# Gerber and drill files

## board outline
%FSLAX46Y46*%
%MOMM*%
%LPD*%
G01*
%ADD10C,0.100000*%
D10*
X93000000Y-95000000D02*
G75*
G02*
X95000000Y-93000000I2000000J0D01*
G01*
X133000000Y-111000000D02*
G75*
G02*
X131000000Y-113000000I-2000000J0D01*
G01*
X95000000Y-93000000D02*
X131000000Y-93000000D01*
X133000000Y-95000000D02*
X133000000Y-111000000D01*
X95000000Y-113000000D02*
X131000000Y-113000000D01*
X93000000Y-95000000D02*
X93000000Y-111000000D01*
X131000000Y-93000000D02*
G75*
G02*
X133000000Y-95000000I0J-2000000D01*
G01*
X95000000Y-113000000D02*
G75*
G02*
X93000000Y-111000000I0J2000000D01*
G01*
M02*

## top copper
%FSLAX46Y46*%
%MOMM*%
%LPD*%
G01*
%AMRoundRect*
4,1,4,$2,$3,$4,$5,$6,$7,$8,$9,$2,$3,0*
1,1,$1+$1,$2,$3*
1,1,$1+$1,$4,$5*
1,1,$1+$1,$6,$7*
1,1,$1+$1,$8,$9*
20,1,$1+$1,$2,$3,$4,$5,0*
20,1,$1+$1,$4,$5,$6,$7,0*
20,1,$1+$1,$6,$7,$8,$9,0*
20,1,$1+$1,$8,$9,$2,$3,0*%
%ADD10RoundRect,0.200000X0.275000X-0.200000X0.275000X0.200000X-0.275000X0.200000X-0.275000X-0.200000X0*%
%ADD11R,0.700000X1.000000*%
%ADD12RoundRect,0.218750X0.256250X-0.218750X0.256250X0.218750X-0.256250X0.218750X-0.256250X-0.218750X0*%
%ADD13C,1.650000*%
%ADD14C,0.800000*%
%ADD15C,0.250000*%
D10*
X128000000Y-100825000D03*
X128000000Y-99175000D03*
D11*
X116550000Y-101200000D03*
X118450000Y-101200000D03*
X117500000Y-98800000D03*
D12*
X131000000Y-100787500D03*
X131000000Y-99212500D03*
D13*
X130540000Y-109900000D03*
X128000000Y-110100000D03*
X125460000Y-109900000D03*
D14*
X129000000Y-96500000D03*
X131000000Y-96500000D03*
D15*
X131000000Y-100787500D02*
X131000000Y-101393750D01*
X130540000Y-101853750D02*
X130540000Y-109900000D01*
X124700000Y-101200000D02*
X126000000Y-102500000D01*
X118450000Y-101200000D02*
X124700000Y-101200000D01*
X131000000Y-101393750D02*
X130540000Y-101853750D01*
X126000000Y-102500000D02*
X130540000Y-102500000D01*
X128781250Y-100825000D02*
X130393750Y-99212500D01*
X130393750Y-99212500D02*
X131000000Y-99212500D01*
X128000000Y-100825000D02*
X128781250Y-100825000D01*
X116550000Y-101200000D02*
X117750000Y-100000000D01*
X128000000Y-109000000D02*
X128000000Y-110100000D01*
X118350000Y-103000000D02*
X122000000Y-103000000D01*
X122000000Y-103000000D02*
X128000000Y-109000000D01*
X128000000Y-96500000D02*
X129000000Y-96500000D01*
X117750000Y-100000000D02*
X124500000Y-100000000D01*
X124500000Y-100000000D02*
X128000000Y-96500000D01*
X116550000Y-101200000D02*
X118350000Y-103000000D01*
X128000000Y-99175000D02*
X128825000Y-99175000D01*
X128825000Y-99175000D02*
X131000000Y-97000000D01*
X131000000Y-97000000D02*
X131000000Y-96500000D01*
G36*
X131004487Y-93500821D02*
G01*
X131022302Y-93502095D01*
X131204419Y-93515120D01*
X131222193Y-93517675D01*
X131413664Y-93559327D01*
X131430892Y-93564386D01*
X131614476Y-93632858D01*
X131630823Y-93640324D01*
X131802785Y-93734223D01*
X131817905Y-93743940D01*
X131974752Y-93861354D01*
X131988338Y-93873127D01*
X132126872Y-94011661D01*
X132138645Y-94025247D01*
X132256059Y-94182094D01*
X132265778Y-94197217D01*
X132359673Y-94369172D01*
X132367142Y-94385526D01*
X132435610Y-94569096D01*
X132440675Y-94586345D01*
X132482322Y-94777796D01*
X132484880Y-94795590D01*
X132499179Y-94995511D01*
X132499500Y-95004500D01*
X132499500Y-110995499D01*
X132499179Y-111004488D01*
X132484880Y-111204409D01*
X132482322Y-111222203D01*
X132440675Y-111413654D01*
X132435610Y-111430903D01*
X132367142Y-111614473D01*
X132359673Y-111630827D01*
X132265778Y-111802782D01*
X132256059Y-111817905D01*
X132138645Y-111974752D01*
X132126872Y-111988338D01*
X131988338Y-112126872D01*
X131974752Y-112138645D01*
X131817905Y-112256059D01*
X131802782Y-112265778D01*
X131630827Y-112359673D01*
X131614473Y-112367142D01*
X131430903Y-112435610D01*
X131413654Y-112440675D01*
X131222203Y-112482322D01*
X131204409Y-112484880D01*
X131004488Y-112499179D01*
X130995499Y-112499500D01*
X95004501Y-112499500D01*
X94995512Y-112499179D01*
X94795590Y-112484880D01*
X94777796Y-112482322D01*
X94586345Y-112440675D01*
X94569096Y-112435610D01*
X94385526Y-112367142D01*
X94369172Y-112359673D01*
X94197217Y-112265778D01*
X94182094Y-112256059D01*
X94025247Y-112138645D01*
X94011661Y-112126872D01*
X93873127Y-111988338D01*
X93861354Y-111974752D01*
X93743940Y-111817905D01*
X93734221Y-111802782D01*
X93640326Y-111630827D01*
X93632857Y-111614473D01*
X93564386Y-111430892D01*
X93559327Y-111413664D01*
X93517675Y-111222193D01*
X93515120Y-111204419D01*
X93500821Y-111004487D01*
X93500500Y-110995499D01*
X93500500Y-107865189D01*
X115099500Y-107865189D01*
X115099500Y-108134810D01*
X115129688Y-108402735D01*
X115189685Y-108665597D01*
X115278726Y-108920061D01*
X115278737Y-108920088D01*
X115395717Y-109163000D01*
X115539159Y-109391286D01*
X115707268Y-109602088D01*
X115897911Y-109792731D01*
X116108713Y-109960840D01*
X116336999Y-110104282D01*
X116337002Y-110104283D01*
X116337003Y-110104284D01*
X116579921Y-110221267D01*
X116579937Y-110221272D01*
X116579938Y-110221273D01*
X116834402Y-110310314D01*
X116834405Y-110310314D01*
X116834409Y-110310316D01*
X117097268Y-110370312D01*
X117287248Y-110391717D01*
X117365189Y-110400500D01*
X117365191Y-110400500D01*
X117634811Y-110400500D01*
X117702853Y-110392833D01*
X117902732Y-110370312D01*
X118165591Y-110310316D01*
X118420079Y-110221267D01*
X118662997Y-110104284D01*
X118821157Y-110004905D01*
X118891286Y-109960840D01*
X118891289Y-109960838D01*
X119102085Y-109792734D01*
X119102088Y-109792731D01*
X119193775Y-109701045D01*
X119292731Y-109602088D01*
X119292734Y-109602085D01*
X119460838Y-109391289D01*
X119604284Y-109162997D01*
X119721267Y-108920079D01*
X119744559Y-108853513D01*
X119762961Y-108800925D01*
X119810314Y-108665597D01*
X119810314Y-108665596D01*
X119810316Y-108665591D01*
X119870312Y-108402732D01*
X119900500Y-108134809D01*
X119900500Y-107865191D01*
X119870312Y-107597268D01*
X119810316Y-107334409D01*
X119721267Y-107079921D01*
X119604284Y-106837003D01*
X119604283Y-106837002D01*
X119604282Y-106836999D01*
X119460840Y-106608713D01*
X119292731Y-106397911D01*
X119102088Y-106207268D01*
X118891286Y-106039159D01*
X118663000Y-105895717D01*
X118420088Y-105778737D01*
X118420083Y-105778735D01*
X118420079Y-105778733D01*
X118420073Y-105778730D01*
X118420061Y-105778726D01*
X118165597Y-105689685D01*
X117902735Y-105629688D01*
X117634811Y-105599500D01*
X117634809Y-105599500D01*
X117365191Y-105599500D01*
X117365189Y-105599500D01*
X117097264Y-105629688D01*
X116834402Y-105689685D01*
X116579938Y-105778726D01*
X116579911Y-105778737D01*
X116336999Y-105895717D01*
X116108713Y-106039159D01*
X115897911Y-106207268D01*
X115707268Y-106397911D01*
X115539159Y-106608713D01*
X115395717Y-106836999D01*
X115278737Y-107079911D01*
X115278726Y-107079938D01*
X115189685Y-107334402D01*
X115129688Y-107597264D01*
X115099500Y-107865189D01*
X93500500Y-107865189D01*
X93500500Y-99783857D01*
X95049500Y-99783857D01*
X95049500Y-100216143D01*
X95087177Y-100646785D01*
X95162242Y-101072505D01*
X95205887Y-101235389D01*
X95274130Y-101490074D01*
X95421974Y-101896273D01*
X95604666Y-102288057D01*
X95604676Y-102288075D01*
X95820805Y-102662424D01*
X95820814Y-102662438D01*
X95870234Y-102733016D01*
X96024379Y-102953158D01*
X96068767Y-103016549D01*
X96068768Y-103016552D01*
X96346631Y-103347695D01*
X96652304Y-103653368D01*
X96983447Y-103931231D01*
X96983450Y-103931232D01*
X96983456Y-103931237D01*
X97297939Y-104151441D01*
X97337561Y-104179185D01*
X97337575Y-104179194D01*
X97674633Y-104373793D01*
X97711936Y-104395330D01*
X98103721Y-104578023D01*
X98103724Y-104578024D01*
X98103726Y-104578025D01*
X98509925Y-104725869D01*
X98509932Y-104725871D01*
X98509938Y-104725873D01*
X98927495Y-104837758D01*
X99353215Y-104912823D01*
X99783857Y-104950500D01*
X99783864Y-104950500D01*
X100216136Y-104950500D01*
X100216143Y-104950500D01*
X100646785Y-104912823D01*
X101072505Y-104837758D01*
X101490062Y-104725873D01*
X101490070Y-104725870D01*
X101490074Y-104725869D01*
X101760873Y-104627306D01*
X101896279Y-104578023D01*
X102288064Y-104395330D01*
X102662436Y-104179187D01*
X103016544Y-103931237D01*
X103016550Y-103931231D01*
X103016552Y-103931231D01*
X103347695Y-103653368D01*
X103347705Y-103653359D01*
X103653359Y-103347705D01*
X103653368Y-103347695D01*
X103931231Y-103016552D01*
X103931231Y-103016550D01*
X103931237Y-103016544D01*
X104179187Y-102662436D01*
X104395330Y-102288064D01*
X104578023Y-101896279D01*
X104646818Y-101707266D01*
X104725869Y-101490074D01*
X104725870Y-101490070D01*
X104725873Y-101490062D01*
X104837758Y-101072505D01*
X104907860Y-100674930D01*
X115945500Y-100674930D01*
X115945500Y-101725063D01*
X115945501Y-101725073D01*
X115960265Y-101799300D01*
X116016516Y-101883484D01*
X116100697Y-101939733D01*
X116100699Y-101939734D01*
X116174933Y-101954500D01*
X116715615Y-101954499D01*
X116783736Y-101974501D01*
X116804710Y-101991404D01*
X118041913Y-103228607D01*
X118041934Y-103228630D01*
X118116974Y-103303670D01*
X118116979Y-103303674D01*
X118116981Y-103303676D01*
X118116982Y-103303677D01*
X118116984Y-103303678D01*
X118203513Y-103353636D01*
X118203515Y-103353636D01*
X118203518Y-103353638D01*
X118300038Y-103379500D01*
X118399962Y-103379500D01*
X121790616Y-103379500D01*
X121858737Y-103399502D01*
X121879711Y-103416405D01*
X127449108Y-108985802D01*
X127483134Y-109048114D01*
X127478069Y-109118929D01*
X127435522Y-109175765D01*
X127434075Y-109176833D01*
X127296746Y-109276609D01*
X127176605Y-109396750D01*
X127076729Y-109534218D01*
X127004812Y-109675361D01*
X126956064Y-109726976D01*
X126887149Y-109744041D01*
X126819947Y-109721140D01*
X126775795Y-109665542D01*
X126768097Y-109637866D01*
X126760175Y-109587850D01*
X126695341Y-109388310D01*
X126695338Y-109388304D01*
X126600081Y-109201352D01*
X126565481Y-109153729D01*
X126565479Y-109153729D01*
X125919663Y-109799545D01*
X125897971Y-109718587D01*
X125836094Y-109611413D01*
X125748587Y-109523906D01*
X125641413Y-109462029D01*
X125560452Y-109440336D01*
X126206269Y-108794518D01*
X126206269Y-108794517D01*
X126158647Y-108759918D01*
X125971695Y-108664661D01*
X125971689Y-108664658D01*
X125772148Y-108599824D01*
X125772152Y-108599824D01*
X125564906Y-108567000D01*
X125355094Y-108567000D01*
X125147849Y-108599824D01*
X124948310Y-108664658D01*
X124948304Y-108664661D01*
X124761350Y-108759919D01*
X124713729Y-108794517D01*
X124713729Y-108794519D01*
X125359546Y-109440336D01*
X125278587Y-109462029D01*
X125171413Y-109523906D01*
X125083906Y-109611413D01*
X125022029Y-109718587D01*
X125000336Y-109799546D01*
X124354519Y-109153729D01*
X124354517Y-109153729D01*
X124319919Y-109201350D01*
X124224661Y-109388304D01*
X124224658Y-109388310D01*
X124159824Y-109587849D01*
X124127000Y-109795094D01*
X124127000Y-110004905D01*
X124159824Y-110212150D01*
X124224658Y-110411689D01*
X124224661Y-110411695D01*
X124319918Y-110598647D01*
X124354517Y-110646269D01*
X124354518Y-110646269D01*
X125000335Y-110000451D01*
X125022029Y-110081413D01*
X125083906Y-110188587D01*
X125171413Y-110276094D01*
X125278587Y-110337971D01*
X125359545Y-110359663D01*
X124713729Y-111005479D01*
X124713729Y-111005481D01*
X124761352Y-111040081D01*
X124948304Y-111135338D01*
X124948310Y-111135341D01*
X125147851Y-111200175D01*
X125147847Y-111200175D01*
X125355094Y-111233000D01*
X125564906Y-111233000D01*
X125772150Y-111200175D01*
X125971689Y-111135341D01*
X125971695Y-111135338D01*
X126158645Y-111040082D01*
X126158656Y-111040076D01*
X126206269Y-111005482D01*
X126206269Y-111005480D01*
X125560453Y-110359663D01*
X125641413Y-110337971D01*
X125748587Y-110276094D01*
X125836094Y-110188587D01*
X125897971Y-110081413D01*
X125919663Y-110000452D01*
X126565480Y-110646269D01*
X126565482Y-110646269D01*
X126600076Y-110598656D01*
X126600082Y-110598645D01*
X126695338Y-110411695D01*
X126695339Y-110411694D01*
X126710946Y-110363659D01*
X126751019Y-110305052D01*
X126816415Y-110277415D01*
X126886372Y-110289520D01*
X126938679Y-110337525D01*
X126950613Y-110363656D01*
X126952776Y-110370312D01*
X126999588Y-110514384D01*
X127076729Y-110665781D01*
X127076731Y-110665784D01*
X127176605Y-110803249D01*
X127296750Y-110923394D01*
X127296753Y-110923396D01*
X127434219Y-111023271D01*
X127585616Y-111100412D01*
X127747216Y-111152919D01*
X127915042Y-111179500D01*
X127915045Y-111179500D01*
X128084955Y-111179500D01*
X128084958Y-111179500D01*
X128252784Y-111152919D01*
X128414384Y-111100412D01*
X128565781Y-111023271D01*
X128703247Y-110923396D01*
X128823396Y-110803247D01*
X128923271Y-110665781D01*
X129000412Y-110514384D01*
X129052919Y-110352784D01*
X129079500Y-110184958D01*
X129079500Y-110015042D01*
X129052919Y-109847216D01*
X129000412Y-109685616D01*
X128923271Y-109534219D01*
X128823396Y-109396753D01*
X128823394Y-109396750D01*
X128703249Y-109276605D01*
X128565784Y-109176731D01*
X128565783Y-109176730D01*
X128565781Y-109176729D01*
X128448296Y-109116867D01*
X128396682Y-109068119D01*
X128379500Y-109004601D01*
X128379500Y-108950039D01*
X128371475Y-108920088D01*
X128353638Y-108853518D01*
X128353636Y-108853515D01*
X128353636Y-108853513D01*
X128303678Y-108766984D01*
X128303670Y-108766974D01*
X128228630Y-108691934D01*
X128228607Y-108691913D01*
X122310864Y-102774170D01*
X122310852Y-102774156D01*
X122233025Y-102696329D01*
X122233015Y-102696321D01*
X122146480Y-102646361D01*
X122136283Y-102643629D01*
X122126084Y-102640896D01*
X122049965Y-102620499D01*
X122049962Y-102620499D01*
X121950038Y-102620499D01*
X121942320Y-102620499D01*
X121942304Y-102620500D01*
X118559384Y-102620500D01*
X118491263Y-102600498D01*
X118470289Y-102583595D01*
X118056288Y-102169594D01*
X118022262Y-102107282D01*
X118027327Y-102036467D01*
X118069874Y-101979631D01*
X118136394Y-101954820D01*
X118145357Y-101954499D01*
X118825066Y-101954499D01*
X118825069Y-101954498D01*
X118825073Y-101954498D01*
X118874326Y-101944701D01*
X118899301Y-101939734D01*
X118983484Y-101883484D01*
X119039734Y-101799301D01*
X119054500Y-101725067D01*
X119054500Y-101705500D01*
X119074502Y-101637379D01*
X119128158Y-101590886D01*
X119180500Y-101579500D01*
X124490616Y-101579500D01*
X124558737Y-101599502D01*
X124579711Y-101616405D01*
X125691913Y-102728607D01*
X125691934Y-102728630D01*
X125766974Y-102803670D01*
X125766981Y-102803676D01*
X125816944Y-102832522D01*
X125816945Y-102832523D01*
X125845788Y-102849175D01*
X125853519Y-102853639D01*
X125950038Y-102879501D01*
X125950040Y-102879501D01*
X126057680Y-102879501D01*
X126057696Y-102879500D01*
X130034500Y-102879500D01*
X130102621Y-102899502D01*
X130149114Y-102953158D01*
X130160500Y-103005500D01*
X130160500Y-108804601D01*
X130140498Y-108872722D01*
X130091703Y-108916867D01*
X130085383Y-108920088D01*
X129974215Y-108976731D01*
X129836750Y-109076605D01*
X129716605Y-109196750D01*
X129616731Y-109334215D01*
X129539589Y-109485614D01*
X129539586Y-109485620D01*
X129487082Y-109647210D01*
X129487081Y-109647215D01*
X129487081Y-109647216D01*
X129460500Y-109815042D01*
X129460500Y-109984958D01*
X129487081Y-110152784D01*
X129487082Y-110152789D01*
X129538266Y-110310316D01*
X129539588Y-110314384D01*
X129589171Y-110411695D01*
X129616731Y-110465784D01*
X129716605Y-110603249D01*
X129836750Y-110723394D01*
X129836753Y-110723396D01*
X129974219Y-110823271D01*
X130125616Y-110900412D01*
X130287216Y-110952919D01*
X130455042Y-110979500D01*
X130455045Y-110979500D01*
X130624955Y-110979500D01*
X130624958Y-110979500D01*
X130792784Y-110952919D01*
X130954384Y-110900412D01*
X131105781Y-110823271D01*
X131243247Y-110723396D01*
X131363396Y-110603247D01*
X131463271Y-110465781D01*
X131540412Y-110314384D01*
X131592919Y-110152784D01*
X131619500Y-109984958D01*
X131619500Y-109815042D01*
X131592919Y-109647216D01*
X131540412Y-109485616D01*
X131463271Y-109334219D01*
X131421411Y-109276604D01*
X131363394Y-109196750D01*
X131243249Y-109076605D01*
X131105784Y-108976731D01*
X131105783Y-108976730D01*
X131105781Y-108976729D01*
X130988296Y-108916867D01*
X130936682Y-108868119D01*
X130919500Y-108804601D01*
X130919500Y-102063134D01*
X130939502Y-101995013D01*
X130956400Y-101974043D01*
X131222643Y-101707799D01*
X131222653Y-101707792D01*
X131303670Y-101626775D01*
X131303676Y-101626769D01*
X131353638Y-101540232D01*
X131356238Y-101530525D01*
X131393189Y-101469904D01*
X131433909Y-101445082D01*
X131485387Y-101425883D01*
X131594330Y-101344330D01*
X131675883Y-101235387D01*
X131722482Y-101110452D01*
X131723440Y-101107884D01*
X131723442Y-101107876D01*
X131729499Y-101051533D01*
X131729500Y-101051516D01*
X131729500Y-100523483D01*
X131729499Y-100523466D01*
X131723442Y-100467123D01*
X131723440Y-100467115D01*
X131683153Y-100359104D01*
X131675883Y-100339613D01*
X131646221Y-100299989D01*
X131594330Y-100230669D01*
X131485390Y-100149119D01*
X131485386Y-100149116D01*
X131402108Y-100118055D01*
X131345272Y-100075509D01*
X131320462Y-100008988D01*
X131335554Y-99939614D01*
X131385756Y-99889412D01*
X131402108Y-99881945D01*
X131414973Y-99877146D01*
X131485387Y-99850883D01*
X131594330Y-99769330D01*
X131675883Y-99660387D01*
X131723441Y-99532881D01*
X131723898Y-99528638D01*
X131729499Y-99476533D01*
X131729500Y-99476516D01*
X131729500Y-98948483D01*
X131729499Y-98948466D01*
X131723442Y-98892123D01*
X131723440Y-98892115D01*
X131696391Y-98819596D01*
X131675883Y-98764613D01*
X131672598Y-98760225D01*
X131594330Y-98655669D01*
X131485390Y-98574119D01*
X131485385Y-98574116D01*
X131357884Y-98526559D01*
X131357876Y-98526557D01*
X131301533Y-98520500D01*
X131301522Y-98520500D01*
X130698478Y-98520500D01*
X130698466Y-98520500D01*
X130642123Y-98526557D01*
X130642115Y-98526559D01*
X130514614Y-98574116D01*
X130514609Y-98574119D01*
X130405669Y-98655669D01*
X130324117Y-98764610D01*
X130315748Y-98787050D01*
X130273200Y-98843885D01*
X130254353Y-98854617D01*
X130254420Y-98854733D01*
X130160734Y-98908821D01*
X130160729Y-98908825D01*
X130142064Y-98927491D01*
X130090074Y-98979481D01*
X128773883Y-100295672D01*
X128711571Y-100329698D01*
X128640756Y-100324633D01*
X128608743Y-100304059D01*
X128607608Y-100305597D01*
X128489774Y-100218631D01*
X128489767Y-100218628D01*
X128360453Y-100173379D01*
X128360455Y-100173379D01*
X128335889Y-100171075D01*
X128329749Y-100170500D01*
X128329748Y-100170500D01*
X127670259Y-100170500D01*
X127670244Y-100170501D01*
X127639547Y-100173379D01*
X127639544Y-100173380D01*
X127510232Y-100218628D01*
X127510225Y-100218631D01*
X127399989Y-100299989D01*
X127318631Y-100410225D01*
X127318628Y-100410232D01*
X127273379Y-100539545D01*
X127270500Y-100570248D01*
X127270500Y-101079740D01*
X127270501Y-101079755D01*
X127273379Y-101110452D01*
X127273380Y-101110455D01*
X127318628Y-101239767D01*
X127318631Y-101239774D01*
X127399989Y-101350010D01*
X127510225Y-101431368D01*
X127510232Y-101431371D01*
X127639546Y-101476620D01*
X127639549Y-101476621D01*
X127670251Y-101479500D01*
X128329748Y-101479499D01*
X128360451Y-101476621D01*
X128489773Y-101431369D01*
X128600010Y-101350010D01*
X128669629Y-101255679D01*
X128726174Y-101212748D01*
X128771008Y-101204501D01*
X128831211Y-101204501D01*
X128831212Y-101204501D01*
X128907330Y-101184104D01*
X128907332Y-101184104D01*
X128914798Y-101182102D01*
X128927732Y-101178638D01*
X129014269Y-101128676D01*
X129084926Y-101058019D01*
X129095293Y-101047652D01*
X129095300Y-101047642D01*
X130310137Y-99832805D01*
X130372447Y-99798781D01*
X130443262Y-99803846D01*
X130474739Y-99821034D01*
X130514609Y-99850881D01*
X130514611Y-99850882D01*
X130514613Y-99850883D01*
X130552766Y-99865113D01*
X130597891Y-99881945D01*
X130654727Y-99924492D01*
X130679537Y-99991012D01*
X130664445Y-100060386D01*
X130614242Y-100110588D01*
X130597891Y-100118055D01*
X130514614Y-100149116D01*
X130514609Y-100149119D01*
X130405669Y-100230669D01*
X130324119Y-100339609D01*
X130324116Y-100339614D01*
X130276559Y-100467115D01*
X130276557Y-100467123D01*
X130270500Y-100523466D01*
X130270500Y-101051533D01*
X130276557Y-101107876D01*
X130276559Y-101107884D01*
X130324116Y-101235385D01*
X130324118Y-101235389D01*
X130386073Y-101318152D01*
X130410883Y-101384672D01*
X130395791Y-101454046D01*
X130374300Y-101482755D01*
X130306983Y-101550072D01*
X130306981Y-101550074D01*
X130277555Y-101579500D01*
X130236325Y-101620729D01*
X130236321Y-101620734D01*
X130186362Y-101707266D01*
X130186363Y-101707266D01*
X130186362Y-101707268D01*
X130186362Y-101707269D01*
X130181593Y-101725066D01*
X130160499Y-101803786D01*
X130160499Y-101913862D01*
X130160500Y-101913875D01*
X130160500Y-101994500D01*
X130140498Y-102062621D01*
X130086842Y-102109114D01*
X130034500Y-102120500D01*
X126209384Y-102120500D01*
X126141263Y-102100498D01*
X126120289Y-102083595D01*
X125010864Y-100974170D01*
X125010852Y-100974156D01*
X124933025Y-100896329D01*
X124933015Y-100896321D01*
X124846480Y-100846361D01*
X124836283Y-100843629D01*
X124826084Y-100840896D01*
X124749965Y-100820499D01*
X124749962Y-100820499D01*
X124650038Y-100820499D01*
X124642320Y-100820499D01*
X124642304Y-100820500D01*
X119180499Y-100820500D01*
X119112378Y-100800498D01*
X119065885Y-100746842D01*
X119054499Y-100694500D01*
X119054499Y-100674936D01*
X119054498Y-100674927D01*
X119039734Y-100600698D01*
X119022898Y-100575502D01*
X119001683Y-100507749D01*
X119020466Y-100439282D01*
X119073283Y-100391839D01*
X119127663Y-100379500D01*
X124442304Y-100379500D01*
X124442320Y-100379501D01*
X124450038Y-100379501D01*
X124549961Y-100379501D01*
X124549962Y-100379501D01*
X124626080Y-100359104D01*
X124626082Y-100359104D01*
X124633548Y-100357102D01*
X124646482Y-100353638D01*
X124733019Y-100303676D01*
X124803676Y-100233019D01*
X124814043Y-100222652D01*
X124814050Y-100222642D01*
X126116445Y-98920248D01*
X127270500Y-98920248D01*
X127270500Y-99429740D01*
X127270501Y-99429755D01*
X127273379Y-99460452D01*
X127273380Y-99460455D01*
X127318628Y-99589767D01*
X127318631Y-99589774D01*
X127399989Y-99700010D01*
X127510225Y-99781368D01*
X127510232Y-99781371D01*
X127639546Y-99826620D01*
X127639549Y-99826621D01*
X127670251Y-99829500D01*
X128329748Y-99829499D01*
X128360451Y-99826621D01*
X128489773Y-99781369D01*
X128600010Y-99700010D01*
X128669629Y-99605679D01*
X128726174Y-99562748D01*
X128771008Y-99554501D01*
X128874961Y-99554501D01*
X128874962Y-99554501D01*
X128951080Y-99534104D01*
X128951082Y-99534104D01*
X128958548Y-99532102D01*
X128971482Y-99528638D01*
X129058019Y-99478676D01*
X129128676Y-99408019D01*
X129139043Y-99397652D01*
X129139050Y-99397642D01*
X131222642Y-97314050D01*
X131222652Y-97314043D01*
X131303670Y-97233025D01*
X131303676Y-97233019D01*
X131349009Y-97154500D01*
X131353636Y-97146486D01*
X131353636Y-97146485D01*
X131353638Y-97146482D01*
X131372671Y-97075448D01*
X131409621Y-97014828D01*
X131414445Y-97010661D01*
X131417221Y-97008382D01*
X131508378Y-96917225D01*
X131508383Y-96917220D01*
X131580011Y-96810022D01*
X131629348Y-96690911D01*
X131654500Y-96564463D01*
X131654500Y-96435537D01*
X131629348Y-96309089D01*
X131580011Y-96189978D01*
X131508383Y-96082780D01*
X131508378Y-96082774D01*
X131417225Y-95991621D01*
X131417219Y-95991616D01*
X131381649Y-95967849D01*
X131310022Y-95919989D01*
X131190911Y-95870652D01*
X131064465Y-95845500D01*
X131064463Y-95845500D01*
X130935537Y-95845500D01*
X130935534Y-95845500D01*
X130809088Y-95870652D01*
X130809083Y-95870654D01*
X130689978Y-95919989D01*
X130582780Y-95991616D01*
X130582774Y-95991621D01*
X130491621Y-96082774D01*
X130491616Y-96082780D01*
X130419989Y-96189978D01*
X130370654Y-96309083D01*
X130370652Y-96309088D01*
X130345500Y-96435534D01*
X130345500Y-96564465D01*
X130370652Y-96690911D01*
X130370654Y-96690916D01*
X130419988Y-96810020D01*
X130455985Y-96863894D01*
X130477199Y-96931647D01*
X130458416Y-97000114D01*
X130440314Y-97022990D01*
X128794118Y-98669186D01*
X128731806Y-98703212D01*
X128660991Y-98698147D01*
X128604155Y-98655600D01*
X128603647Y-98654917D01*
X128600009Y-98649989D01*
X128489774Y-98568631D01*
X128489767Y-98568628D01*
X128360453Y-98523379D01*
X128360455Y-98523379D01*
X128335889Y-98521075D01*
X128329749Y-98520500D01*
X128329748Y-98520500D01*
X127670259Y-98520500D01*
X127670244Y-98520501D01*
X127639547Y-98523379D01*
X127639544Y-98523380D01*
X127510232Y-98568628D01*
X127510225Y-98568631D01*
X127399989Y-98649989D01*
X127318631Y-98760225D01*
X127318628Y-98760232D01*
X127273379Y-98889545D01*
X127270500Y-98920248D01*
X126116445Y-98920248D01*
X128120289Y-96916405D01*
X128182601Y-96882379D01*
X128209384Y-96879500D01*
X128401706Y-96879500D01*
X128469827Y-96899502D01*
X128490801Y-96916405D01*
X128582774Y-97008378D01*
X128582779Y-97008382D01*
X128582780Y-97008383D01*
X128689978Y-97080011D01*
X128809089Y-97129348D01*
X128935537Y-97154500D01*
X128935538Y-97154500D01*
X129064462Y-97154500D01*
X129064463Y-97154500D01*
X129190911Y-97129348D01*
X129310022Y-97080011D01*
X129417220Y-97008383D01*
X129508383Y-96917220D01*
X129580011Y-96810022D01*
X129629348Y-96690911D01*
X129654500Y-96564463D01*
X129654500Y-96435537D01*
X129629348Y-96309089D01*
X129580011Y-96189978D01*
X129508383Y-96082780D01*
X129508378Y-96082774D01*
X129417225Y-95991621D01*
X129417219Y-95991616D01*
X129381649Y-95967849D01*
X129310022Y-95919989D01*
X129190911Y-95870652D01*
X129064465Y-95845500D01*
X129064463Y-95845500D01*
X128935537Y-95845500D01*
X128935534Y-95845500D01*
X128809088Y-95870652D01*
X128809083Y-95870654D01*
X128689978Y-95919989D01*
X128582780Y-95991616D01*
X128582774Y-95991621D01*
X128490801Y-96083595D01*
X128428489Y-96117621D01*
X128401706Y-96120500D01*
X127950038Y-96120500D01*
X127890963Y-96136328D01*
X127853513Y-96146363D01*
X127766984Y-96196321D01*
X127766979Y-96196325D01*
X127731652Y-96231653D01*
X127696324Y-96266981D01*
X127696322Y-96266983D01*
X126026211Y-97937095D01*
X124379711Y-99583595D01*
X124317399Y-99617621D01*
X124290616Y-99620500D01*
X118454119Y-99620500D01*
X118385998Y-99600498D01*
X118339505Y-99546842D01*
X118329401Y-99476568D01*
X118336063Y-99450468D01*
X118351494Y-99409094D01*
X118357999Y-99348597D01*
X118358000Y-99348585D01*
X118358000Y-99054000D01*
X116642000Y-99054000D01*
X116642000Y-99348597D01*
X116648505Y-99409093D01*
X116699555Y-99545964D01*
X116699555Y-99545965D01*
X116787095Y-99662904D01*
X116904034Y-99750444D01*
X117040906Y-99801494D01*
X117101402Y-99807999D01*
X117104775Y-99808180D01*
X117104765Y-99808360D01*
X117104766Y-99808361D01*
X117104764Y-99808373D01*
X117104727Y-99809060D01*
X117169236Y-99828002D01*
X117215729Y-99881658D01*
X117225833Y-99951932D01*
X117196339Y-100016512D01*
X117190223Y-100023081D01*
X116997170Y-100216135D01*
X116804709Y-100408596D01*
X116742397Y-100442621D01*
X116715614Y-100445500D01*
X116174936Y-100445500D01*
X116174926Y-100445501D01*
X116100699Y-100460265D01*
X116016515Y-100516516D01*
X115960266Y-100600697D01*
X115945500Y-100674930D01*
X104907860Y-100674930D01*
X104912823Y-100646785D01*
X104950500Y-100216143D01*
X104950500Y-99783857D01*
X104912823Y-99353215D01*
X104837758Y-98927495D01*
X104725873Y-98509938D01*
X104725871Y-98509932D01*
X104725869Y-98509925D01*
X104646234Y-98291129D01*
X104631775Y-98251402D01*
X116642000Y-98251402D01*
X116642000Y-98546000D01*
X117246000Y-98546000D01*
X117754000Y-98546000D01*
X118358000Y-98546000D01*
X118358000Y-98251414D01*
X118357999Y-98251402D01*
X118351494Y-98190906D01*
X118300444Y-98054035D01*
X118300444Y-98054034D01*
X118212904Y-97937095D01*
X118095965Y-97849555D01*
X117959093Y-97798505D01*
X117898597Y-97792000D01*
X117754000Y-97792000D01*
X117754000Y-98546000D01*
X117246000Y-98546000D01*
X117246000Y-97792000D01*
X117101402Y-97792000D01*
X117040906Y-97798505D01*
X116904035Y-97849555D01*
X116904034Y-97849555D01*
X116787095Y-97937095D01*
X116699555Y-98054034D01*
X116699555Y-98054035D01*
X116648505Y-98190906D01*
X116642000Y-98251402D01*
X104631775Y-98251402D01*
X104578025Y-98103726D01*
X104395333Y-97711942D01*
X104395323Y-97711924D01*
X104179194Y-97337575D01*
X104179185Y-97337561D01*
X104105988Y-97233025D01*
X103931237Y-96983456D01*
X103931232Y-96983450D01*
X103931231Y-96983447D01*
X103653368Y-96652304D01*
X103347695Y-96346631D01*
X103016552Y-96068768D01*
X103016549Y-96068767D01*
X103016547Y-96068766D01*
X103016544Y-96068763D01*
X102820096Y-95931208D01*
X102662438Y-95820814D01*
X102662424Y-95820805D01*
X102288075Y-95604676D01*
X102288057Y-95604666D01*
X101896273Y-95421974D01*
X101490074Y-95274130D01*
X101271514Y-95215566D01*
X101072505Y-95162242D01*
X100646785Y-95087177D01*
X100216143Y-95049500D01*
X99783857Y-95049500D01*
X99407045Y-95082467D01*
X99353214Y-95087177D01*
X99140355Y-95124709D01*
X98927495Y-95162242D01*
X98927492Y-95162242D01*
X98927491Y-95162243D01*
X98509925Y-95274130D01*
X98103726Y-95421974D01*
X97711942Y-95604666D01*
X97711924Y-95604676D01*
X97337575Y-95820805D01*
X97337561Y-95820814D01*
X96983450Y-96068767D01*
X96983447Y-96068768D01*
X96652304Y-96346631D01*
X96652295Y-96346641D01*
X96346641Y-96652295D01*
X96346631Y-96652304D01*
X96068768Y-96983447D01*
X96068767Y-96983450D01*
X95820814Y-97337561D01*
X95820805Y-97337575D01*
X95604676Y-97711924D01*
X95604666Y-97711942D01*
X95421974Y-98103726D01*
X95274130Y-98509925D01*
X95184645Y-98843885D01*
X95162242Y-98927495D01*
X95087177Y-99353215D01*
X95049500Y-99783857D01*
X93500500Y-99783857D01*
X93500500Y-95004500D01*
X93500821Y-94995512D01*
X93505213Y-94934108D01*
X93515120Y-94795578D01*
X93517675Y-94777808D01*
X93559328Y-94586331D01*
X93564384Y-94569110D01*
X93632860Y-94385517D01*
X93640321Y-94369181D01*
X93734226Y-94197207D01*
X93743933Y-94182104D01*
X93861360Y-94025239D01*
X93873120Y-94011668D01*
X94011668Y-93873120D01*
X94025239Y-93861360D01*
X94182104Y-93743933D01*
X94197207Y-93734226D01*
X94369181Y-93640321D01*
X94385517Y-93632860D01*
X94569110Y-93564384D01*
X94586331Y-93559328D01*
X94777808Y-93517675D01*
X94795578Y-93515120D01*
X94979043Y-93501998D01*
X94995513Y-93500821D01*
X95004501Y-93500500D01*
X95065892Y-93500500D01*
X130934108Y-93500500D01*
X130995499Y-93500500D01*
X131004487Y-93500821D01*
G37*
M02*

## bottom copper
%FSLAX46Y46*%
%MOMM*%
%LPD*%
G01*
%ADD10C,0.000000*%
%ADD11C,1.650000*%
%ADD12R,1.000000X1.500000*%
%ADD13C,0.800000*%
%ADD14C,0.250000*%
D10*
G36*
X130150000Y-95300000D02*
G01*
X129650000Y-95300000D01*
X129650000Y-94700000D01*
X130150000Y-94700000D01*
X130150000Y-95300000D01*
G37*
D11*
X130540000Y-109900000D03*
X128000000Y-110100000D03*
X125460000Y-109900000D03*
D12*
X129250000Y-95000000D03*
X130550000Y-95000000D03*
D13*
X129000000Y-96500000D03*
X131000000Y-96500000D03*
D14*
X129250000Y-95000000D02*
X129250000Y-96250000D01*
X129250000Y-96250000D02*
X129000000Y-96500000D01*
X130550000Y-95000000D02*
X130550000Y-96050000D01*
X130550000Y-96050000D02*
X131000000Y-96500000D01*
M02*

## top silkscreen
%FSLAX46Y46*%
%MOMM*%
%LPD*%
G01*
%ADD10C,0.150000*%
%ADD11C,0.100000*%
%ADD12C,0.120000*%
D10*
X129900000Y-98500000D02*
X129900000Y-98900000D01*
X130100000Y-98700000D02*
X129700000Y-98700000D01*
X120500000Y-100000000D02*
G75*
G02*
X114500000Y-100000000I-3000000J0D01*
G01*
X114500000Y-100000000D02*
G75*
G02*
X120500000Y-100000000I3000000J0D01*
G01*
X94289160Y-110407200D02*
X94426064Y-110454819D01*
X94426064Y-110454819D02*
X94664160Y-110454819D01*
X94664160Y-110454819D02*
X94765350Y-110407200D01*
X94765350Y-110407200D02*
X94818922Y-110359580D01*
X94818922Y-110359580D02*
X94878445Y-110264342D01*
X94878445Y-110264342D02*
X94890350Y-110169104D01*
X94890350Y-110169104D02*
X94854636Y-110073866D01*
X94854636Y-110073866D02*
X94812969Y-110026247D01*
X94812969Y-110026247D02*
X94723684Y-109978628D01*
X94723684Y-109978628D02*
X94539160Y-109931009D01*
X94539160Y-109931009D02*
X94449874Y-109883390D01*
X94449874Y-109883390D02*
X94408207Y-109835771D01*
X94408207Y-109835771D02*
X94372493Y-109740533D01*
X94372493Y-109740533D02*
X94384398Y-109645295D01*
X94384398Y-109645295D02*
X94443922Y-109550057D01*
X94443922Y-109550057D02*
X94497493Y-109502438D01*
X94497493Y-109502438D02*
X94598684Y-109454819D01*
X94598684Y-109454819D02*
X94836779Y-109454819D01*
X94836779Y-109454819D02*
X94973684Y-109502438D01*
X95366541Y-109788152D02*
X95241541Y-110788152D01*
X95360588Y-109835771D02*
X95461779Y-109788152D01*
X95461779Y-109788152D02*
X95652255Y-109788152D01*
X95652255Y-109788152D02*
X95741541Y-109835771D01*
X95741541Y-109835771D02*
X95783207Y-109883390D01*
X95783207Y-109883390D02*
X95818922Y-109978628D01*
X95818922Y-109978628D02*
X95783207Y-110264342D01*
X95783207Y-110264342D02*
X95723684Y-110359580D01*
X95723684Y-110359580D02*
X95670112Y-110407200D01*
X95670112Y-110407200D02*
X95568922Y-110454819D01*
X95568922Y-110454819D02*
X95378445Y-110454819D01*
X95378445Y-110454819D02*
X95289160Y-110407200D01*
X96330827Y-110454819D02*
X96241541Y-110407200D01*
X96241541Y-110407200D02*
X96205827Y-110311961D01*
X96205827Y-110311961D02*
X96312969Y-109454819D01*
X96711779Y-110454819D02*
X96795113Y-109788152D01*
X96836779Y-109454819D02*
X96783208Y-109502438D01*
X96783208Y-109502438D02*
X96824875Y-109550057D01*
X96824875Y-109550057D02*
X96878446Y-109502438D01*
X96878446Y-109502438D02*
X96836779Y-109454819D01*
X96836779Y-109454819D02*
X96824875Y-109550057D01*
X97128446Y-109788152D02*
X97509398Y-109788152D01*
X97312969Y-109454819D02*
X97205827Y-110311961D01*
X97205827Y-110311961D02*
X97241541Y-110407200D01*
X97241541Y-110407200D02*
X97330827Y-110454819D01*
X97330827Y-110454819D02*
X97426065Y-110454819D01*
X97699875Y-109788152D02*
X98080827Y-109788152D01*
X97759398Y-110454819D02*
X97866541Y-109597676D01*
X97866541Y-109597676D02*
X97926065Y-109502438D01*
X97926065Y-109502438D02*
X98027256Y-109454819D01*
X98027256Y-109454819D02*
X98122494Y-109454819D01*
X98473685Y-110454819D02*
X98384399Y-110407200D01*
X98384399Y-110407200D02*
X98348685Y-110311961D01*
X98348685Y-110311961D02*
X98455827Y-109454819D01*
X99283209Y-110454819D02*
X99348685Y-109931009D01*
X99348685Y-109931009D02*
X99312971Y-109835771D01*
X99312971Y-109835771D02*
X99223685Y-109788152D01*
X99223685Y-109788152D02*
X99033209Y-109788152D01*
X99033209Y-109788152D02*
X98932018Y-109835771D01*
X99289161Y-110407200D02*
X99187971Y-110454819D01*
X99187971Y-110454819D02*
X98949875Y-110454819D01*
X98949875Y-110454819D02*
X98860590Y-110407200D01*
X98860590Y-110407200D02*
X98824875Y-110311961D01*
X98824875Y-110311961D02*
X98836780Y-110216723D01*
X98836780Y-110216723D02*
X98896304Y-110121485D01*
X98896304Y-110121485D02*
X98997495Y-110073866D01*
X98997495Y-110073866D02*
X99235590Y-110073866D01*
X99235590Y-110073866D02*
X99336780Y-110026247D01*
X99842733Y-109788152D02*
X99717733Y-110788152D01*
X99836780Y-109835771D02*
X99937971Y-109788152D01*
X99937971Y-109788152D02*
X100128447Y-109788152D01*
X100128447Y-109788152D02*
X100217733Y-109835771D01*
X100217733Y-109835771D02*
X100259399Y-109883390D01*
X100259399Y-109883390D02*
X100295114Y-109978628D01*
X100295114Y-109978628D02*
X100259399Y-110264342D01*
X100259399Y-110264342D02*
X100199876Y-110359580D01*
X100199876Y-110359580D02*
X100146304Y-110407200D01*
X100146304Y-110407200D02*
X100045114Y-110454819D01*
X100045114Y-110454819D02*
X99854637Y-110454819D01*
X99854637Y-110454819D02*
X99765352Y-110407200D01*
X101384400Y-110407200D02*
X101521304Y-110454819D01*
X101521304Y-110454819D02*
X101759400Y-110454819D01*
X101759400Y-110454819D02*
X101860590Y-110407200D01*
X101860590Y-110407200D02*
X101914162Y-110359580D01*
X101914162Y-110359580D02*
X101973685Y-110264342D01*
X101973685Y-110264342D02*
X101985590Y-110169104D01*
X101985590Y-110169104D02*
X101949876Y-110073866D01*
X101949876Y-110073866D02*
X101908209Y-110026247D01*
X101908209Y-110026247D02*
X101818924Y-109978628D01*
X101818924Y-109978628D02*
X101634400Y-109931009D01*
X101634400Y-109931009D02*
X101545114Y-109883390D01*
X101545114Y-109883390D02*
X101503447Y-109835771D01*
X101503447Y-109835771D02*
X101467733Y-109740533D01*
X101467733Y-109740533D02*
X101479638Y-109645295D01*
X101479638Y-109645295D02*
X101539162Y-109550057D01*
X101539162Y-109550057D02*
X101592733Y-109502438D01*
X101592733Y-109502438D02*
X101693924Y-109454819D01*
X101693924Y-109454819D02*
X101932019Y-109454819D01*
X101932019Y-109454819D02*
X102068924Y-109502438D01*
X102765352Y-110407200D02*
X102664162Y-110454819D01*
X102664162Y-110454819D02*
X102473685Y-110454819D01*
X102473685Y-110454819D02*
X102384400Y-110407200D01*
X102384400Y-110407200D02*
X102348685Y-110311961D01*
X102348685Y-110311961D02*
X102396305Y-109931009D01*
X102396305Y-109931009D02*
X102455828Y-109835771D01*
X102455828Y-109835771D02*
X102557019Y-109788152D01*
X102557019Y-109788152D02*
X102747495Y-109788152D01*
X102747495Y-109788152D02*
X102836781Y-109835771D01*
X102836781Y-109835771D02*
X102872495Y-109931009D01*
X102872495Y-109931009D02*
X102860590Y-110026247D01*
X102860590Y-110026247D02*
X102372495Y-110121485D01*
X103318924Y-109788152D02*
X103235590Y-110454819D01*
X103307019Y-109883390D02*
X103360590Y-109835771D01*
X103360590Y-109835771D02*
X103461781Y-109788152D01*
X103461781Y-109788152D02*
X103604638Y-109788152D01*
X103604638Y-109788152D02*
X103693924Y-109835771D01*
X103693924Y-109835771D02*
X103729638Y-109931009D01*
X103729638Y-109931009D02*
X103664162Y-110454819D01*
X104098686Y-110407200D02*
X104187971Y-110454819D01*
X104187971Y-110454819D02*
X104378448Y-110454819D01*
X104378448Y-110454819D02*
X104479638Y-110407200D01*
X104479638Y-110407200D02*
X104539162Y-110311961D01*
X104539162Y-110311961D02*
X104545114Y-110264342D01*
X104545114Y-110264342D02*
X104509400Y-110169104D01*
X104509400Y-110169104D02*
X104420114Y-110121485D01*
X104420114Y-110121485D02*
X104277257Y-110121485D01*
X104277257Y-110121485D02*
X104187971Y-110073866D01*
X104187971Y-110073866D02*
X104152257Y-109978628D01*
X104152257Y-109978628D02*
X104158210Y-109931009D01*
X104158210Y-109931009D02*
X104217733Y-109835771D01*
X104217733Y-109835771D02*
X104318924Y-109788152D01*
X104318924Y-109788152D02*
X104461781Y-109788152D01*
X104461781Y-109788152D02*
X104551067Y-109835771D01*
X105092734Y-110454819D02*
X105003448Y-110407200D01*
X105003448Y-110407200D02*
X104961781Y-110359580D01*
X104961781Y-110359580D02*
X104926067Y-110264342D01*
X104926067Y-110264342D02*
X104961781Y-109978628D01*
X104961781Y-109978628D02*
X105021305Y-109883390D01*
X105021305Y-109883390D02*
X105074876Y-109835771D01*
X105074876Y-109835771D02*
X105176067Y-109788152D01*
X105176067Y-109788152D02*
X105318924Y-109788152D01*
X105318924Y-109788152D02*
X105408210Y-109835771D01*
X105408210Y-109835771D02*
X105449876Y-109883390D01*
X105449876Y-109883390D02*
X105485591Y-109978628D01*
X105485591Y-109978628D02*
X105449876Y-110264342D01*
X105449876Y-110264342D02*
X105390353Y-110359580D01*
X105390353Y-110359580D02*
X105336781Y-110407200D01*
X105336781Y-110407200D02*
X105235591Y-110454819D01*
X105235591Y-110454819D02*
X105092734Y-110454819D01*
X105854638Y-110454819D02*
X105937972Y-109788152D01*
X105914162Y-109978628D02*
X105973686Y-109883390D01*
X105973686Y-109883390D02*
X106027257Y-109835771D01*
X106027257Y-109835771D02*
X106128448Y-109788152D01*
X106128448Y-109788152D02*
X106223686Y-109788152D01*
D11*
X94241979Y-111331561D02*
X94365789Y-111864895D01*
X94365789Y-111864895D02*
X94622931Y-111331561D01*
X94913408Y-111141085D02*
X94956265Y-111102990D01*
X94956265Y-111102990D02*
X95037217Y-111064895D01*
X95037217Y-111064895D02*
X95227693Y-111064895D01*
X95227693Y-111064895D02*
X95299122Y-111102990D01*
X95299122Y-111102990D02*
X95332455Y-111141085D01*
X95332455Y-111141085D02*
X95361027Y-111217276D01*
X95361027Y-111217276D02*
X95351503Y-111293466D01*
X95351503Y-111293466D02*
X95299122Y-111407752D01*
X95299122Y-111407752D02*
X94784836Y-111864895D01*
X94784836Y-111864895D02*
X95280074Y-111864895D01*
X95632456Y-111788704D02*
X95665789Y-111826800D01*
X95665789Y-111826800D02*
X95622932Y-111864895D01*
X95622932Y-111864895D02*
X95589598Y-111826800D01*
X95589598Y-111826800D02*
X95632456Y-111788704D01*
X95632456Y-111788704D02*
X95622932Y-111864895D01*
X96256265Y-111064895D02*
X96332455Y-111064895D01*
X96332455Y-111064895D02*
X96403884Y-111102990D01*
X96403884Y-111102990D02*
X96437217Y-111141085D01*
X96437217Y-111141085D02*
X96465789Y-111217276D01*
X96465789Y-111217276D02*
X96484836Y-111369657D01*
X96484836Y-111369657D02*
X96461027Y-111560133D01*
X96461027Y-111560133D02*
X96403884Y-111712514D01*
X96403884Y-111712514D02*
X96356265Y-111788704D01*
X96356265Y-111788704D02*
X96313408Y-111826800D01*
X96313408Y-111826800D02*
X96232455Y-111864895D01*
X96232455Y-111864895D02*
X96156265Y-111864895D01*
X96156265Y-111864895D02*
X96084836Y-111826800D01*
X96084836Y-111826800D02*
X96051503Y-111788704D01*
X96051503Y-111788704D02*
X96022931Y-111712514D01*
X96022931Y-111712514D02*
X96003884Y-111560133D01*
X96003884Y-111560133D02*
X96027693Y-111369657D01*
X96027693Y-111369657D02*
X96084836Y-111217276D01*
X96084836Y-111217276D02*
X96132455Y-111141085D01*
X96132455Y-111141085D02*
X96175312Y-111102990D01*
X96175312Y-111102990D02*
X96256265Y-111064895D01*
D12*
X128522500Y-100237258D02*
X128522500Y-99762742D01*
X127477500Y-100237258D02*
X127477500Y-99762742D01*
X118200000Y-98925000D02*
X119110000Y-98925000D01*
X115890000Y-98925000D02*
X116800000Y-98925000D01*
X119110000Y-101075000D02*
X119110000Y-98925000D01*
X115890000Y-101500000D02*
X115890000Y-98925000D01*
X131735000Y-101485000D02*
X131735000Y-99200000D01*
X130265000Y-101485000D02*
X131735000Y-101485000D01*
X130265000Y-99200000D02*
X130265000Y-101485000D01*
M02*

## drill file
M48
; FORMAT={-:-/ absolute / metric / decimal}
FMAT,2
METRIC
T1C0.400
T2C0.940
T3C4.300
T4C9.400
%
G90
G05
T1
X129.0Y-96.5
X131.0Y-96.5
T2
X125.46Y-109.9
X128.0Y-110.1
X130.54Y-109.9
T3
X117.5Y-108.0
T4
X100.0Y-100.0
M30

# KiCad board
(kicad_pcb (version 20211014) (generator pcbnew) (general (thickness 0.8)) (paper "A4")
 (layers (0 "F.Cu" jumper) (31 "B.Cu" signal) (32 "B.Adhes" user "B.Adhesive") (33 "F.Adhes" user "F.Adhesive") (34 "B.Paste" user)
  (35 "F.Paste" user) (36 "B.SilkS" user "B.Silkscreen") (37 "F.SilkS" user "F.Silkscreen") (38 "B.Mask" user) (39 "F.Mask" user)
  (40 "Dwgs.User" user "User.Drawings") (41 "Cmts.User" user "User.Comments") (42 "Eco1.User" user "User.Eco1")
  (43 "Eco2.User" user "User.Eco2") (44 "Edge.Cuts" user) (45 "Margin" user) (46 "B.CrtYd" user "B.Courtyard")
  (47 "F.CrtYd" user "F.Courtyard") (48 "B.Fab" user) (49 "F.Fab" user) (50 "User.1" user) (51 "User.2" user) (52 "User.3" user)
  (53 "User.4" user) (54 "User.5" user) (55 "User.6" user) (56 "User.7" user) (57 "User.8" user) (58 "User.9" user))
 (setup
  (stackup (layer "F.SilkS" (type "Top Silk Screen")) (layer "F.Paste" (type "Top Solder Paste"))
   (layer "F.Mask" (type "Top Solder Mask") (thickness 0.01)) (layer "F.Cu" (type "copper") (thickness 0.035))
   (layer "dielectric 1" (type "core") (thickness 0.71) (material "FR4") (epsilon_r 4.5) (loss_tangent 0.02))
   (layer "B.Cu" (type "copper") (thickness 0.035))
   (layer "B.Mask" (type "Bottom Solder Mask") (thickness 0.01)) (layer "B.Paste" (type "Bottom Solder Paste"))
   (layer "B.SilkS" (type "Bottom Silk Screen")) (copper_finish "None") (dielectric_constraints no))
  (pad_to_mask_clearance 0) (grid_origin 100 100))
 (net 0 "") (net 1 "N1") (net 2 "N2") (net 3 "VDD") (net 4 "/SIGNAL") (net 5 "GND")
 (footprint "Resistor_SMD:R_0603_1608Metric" (layer "F.Cu") (at 128 100 90)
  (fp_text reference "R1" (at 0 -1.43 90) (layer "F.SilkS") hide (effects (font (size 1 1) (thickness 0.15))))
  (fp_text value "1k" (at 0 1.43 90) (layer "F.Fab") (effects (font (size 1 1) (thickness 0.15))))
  (fp_line (start -0.237258 0.5225) (end 0.237258 0.5225) (layer "F.SilkS") (width 0.12))
  (fp_line (start -0.237258 -0.5225) (end 0.237258 -0.5225) (layer "F.SilkS") (width 0.12))
  (pad "1" smd roundrect (at -0.825 0 90) (size 0.8 0.95) (layers "F.Cu" "F.Paste" "F.Mask") (roundrect_rratio 0.25) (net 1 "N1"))
  (pad "2" smd roundrect (at 0.825 0 90) (size 0.8 0.95) (layers "F.Cu" "F.Paste" "F.Mask") (roundrect_rratio 0.25) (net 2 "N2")))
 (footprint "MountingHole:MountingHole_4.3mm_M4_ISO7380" (layer "F.Cu") (at 117.5 108)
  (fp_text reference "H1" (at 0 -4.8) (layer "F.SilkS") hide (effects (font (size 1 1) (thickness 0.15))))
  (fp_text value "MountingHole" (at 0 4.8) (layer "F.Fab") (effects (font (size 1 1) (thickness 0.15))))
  (pad "" np_thru_hole circle (at 0 0) (size 4.3 4.3) (drill 4.3) (layers *.Cu *.Mask)))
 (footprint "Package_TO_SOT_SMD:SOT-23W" (layer "F.Cu") (at 117.5 100 90)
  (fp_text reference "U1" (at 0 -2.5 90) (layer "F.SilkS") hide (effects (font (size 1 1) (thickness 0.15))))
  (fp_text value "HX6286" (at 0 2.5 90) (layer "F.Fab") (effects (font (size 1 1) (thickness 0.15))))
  (fp_line (start 1.075 0.7) (end 1.075 1.61) (layer "F.SilkS") (width 0.12))
  (fp_line (start 1.075 -1.61) (end 1.075 -0.7) (layer "F.SilkS") (width 0.12))
  (fp_line (start -1.075 1.61) (end 1.075 1.61) (layer "F.SilkS") (width 0.12))
  (fp_line (start -1.5 -1.61) (end 1.075 -1.61) (layer "F.SilkS") (width 0.12))
  (pad "1" smd rect (at -1.2 -0.95 90) (size 1 0.7) (layers "F.Cu" "F.Paste" "F.Mask") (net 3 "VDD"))
  (pad "2" smd rect (at -1.2 0.95 90) (size 1 0.7) (layers "F.Cu" "F.Paste" "F.Mask") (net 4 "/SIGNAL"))
  (pad "3" smd rect (at 1.2 0 90) (size 1 0.7) (layers "F.Cu" "F.Paste" "F.Mask") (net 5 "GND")))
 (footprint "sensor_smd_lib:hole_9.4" (layer "F.Cu") (at 100 100)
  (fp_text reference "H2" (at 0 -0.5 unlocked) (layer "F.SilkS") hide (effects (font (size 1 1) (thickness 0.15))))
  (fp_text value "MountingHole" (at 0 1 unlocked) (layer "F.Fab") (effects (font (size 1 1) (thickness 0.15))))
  (pad "" np_thru_hole circle (at 0 0) (size 9.4 9.4) (drill 9.4) (layers F&B.Cu *.Mask)))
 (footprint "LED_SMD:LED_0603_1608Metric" (layer "F.Cu") (at 131 100 90)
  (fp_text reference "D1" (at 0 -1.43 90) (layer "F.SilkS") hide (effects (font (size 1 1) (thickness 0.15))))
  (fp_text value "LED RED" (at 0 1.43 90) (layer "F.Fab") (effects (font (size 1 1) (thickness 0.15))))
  (fp_line (start -1.485 0.735) (end 0.8 0.735) (layer "F.SilkS") (width 0.12))
  (fp_line (start -1.485 -0.735) (end -1.485 0.735) (layer "F.SilkS") (width 0.12))
  (fp_line (start 0.8 -0.735) (end -1.485 -0.735) (layer "F.SilkS") (width 0.12))
  (pad "1" smd roundrect (at -0.7875 0 90) (size 0.875 0.95) (layers "F.Cu" "F.Paste" "F.Mask") (roundrect_rratio 0.25) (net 4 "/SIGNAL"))
  (pad "2" smd roundrect (at 0.7875 0 90) (size 0.875 0.95) (layers "F.Cu" "F.Paste" "F.Mask") (roundrect_rratio 0.25) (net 1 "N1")))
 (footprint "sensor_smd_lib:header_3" (layer "B.Cu") (at 128 113 180)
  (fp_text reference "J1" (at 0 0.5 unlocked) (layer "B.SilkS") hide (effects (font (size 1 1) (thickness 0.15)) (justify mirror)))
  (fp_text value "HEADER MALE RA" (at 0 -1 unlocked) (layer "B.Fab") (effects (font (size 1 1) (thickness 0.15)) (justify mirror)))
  (pad "1" thru_hole circle (at -2.54 3.1 180) (size 1.65 1.65) (drill 0.94) (layers *.Cu *.Mask) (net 4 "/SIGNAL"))
  (pad "2" thru_hole circle (at 0 2.9 180) (size 1.65 1.65) (drill 0.94) (layers *.Cu *.Mask) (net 3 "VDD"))
  (pad "3" thru_hole circle (at 2.54 3.1 180) (size 1.65 1.65) (drill 0.94) (layers *.Cu *.Mask) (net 5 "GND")))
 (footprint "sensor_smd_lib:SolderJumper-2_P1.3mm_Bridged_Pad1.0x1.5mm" (layer "B.Cu") (at 129.9 95)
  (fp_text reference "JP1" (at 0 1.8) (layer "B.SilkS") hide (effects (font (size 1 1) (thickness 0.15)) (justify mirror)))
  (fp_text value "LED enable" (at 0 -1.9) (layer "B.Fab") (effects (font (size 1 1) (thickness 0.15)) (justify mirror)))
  (fp_poly (pts (xy -0.25 0.3) (xy 0.25 0.3) (xy 0.25 -0.3) (xy -0.25 -0.3)) (layer "B.Cu") (width 0) (fill solid))
  (pad "1" smd rect (at -0.65 0) (size 1 1.5) (layers "B.Cu" "B.Mask") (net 3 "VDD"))
  (pad "2" smd rect (at 0.65 0) (size 1 1.5) (layers "B.Cu" "B.Mask") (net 2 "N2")))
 (gr_line (start 129.9 98.5) (end 129.9 98.9) (layer "F.SilkS") (width 0.15))
 (gr_line (start 130.1 98.7) (end 129.7 98.7) (layer "F.SilkS") (width 0.15))
 (gr_circle (center 117.5 100) (end 120.5 100) (layer "F.SilkS") (width 0.15) (fill none))
 (gr_arc (start 93 95) (mid 93.585786 93.585786) (end 95 93) (layer "Edge.Cuts") (width 0.1))
 (gr_arc (start 133 111) (mid 132.414214 112.414214) (end 131 113) (layer "Edge.Cuts") (width 0.1))
 (gr_line (start 95 93) (end 131 93) (layer "Edge.Cuts") (width 0.1))
 (gr_line (start 133 95) (end 133 111) (layer "Edge.Cuts") (width 0.1))
 (gr_line (start 95 113) (end 131 113) (layer "Edge.Cuts") (width 0.1))
 (gr_line (start 93 95) (end 93 111) (layer "Edge.Cuts") (width 0.1))
 (gr_arc (start 131 93) (mid 132.414214 93.585786) (end 133 95) (layer "Edge.Cuts") (width 0.1))
 (gr_arc (start 95 113) (mid 93.585786 112.414214) (end 93 111) (layer "Edge.Cuts") (width 0.1))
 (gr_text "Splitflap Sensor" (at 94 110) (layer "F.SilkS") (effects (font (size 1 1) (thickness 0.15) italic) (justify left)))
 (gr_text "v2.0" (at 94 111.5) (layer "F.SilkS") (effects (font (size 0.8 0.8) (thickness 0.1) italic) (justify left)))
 (segment (start 131 100.7875) (end 131 101.39375) (width 0.25) (layer "F.Cu") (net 4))
 (segment (start 130.54 101.85375) (end 130.54 109.9) (width 0.25) (layer "F.Cu") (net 4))
 (segment (start 124.7 101.2) (end 126 102.5) (width 0.25) (layer "F.Cu") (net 4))
 (segment (start 118.45 101.2) (end 124.7 101.2) (width 0.25) (layer "F.Cu") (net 4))
 (segment (start 131 101.39375) (end 130.54 101.85375) (width 0.25) (layer "F.Cu") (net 4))
 (segment (start 126 102.5) (end 130.54 102.5) (width 0.25) (layer "F.Cu") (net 4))
 (segment (start 128.78125 100.825) (end 130.39375 99.2125) (width 0.25) (layer "F.Cu") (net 1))
 (segment (start 130.39375 99.2125) (end 131 99.2125) (width 0.25) (layer "F.Cu") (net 1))
 (segment (start 128 100.825) (end 128.78125 100.825) (width 0.25) (layer "F.Cu") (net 1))
 (segment (start 116.55 101.2) (end 117.75 100) (width 0.25) (layer "F.Cu") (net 3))
 (segment (start 128 109) (end 128 110.1) (width 0.25) (layer "F.Cu") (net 3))
 (segment (start 118.35 103) (end 122 103) (width 0.25) (layer "F.Cu") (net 3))
 (segment (start 122 103) (end 128 109) (width 0.25) (layer "F.Cu") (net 3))
 (segment (start 128 96.5) (end 129 96.5) (width 0.25) (layer "F.Cu") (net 3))
 (segment (start 117.75 100) (end 124.5 100) (width 0.25) (layer "F.Cu") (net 3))
 (segment (start 124.5 100) (end 128 96.5) (width 0.25) (layer "F.Cu") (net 3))
 (segment (start 116.55 101.2) (end 118.35 103) (width 0.25) (layer "F.Cu") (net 3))
 (via (at 129 96.5) (size 0.8) (drill 0.4) (layers "F.Cu" "B.Cu") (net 3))
 (segment (start 129.25 95) (end 129.25 96.25) (width 0.25) (layer "B.Cu") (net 3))
 (segment (start 129.25 96.25) (end 129 96.5) (width 0.25) (layer "B.Cu") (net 3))
 (segment (start 128 99.175) (end 128.825 99.175) (width 0.25) (layer "F.Cu") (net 2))
 (segment (start 128.825 99.175) (end 131 97) (width 0.25) (layer "F.Cu") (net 2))
 (segment (start 131 97) (end 131 96.5) (width 0.25) (layer "F.Cu") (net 2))
 (via (at 131 96.5) (size 0.8) (drill 0.4) (layers "F.Cu" "B.Cu") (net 2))
 (segment (start 130.55 95) (end 130.55 96.05) (width 0.25) (layer "B.Cu") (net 2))
 (segment (start 130.55 96.05) (end 131 96.5) (width 0.25) (layer "B.Cu") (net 2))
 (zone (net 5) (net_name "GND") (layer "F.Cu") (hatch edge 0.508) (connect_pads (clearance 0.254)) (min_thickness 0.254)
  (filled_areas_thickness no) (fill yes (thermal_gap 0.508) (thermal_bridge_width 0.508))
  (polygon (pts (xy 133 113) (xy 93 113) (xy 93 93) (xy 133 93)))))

